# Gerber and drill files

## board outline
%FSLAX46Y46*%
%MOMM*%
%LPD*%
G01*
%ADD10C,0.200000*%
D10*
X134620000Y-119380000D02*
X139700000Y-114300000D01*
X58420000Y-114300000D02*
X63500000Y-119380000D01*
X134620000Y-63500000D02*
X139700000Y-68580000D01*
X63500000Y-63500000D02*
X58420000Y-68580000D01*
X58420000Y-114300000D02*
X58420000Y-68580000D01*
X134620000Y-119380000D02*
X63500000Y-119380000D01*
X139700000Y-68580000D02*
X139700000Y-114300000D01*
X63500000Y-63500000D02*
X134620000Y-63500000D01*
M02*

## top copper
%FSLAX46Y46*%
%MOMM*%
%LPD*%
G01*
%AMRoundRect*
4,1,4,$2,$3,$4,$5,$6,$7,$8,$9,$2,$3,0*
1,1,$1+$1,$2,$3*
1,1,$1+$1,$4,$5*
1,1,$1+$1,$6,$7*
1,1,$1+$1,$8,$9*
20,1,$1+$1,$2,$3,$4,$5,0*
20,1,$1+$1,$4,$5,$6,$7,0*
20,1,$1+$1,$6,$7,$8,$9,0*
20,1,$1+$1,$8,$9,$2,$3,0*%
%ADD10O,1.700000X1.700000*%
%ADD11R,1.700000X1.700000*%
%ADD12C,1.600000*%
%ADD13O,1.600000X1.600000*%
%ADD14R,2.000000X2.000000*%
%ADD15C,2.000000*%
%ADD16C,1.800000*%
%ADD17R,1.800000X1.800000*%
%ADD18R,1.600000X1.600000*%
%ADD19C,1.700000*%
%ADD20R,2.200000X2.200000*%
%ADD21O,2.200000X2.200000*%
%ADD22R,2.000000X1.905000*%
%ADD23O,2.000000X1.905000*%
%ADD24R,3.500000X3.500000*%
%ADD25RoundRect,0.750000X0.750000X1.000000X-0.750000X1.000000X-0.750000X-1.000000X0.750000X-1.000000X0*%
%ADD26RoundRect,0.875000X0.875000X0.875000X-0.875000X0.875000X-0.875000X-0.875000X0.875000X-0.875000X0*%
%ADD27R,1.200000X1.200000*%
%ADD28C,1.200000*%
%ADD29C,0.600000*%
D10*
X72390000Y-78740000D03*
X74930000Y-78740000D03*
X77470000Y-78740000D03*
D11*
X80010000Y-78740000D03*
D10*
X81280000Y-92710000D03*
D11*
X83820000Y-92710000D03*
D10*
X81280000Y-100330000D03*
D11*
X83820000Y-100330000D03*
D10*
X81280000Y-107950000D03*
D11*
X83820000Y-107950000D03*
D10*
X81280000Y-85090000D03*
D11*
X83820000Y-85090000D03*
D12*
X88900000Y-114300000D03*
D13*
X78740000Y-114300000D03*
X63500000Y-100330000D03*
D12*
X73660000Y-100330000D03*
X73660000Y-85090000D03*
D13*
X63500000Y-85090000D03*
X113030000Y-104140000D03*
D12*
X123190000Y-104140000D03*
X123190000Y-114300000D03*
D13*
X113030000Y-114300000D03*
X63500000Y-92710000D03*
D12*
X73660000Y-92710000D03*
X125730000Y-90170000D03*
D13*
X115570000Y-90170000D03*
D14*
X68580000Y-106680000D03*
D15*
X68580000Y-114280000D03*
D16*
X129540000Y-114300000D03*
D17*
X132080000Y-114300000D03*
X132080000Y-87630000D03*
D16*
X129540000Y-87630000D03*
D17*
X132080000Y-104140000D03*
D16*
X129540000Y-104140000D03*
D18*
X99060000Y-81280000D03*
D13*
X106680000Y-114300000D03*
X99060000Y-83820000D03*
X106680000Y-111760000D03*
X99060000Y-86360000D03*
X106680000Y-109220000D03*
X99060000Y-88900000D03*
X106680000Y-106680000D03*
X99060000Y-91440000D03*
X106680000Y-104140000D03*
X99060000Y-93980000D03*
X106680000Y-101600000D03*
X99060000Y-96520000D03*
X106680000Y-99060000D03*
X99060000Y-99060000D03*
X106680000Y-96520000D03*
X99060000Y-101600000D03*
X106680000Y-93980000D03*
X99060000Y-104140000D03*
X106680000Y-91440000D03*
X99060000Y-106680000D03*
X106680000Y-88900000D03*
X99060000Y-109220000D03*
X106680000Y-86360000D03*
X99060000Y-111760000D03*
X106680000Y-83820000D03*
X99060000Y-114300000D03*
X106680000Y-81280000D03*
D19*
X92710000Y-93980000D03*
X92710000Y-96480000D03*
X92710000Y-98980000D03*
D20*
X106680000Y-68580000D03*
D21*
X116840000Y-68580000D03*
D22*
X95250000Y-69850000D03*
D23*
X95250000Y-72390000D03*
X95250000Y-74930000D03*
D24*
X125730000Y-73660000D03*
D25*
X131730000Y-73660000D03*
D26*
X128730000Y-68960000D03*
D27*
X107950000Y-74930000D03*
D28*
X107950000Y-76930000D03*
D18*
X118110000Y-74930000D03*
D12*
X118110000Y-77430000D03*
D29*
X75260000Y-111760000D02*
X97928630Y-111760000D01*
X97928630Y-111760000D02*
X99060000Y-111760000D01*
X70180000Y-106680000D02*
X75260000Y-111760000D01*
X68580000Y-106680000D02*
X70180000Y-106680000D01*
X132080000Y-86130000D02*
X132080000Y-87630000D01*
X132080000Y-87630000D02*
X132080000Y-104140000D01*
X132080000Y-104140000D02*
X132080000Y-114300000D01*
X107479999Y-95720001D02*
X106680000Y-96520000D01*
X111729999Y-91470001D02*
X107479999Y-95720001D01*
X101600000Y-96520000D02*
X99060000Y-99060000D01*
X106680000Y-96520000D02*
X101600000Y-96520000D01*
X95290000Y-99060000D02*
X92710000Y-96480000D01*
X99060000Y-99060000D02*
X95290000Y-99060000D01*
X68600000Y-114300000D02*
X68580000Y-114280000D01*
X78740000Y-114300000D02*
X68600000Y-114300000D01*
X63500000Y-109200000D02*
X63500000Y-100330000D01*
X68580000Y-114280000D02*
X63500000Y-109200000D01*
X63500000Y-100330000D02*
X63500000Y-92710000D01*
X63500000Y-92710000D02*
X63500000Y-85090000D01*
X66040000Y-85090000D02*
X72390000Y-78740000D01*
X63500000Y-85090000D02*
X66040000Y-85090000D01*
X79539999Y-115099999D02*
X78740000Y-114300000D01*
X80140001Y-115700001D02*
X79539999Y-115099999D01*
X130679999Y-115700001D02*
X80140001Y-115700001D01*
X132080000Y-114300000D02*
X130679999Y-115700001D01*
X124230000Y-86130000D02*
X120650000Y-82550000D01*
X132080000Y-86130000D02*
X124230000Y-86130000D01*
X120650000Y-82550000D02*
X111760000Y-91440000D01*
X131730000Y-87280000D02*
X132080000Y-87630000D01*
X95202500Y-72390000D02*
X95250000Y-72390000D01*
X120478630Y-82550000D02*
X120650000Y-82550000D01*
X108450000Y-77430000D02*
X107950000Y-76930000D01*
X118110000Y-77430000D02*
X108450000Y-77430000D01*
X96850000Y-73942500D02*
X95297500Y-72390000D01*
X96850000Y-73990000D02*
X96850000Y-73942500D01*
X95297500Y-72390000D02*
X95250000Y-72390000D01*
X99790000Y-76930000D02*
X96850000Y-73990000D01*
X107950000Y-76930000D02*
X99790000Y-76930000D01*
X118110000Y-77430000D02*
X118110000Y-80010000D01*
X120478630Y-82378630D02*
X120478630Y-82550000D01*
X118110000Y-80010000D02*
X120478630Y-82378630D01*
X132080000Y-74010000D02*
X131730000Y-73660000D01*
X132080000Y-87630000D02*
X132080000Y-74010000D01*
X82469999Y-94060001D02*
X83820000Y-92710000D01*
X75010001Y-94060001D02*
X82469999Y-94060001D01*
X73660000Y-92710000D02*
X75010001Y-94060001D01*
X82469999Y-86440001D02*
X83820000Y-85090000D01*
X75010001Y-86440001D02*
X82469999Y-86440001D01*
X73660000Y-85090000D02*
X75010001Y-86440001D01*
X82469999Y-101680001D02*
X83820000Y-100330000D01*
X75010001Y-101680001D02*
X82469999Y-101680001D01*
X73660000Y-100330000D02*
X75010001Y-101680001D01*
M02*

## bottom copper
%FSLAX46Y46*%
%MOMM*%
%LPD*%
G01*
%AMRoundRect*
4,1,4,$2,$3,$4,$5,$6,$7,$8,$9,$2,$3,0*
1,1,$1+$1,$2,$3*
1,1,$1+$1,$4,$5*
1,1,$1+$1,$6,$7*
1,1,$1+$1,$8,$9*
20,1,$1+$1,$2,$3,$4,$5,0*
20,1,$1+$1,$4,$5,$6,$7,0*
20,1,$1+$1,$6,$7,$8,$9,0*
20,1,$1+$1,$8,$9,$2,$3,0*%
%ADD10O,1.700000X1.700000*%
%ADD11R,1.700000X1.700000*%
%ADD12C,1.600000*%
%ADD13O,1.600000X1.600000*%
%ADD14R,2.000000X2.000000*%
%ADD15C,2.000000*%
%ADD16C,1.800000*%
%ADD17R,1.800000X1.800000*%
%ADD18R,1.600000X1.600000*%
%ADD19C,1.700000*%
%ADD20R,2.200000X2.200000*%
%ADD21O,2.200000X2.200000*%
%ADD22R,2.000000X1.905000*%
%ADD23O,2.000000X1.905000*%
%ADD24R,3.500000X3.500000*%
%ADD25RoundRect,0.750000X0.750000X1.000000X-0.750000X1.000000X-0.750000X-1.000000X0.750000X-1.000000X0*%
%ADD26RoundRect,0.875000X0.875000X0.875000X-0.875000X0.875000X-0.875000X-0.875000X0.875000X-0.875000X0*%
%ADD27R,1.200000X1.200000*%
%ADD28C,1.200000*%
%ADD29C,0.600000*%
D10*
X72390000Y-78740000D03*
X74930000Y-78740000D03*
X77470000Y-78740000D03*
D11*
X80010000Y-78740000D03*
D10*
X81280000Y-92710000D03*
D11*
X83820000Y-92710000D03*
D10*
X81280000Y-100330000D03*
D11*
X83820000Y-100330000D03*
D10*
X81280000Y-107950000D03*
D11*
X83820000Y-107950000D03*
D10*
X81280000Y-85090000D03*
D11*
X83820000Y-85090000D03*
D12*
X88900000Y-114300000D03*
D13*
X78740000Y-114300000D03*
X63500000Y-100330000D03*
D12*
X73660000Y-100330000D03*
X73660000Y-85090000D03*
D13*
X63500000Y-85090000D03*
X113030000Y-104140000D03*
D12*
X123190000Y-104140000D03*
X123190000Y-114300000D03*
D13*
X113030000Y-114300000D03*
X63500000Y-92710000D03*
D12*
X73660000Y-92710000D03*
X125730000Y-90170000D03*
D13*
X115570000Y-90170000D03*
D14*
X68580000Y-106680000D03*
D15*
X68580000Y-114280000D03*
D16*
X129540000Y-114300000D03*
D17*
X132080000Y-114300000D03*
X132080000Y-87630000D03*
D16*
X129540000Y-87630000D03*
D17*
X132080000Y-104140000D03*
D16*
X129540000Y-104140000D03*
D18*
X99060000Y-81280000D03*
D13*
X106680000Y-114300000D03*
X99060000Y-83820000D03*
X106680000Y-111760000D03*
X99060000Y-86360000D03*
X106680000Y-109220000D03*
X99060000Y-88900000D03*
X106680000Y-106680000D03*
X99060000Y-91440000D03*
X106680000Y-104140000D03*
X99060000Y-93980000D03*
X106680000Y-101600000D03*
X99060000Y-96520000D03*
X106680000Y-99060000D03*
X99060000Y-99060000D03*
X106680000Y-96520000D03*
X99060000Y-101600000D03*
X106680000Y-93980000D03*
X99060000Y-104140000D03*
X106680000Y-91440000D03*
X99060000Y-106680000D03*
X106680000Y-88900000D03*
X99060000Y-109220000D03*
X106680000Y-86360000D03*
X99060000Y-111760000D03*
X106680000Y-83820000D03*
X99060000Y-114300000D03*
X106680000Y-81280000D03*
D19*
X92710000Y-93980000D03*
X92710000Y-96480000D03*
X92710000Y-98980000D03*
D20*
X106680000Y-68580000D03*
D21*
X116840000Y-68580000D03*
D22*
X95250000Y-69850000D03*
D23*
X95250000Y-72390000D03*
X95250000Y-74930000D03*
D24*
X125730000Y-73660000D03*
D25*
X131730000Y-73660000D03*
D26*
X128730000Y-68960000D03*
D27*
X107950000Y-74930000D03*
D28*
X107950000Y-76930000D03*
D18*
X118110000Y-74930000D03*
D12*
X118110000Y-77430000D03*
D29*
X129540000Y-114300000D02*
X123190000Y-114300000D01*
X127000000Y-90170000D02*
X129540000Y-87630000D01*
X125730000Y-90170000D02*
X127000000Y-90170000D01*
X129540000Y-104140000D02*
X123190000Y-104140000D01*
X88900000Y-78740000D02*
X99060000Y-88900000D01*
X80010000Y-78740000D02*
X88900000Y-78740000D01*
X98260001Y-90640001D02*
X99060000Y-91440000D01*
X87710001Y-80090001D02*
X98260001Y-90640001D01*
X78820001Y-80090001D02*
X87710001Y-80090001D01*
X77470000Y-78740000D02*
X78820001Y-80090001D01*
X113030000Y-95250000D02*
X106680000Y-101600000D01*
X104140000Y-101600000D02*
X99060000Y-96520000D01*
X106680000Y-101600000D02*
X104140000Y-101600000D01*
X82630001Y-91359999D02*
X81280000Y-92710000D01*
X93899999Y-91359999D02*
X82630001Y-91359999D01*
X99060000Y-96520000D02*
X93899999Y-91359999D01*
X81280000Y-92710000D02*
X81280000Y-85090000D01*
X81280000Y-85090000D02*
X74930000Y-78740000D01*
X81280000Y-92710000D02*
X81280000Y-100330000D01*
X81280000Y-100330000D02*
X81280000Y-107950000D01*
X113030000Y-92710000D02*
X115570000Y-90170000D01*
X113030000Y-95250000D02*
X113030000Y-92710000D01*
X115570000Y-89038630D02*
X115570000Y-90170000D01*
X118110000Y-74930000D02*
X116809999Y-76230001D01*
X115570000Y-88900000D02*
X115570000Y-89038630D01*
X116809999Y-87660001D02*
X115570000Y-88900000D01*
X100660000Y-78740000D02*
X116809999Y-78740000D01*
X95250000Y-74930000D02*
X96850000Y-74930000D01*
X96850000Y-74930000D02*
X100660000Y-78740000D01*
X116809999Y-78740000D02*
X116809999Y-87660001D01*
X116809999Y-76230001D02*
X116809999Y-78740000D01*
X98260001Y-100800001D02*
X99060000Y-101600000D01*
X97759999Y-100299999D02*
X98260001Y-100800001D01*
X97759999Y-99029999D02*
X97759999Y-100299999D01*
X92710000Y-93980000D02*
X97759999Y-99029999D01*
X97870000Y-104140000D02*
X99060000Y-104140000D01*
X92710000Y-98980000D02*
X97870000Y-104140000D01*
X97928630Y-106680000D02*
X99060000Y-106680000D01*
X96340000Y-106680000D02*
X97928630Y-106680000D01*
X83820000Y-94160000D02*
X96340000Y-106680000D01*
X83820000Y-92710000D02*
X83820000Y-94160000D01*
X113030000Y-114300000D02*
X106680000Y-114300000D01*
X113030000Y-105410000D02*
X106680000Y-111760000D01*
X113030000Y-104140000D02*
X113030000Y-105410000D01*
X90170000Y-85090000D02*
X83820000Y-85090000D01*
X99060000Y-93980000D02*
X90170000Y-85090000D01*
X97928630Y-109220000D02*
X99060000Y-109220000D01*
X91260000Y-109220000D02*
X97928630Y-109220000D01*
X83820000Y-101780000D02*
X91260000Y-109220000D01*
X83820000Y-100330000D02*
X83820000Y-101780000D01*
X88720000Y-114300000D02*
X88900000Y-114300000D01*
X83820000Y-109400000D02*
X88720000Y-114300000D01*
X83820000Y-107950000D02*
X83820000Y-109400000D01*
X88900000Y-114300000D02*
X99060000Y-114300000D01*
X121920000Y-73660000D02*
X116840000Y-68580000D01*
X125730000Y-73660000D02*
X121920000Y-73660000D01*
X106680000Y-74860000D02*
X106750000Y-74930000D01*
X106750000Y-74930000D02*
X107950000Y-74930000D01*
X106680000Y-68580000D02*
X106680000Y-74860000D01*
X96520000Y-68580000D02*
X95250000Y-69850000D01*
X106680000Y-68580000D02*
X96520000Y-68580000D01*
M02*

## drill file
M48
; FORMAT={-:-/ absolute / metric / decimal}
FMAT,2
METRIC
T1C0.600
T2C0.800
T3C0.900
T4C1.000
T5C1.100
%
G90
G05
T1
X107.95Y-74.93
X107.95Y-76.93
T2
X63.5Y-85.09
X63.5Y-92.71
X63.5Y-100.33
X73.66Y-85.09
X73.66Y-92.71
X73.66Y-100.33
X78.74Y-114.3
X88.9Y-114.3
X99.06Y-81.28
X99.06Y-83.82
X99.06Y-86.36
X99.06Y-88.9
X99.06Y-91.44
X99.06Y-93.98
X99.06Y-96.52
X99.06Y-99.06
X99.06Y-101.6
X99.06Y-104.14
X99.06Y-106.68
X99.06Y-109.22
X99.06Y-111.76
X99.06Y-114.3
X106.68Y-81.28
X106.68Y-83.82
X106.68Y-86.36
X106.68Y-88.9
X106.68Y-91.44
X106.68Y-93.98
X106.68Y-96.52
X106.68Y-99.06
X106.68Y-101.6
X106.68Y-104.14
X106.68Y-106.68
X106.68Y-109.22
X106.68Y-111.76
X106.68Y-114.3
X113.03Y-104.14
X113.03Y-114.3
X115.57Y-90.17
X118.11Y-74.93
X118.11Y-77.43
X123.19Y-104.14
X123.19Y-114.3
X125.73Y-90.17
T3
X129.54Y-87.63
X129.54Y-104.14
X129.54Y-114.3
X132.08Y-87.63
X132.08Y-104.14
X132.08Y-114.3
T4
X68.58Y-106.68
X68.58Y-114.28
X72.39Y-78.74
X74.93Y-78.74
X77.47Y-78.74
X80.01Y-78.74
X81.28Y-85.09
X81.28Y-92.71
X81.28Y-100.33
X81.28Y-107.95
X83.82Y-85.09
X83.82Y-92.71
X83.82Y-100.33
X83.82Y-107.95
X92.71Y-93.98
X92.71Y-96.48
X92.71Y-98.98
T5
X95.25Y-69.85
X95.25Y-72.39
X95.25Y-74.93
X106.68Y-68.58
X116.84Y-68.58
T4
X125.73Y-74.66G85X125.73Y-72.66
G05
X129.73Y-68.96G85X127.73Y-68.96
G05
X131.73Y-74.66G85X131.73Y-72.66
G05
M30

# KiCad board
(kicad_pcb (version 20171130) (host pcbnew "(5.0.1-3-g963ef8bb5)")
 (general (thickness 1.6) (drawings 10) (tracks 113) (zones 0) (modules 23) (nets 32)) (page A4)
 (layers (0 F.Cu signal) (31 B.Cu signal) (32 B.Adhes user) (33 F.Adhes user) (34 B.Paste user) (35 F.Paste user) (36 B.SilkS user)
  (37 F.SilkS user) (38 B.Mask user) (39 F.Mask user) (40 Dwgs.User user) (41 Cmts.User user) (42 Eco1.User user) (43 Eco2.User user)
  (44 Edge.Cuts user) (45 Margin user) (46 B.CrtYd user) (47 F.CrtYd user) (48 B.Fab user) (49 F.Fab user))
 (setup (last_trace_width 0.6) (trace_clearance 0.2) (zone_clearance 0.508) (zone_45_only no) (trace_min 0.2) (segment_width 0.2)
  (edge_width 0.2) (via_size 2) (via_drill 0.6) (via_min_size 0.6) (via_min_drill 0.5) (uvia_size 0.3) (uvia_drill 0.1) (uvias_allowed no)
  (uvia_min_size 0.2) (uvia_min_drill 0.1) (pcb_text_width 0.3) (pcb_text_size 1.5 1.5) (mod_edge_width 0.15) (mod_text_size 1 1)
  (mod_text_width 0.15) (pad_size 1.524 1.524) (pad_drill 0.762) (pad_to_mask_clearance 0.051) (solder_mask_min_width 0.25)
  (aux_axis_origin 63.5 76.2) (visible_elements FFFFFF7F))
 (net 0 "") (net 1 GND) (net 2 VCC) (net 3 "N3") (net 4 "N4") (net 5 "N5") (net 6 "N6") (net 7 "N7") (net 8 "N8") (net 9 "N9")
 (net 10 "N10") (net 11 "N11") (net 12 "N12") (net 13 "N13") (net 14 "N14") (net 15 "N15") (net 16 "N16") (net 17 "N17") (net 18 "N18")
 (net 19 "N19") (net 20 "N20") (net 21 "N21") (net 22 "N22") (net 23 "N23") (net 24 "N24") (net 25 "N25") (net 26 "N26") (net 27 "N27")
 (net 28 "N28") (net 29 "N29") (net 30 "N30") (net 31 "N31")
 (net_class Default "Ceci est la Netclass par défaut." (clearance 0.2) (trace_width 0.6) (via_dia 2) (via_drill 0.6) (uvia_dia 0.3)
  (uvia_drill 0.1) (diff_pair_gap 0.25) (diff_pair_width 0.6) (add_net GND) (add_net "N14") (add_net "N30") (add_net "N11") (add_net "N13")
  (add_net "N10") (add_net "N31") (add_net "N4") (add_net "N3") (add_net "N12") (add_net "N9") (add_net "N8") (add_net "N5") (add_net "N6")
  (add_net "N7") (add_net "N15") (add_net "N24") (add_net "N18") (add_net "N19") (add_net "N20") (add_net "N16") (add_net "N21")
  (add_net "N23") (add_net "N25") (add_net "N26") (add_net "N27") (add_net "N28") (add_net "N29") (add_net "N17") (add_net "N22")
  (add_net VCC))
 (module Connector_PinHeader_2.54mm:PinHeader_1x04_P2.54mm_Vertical (layer F.Cu) (at 80.01 78.74 270)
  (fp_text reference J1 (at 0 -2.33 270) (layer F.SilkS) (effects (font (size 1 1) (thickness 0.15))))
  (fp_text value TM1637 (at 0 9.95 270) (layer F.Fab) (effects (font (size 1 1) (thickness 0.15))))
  (pad 4 thru_hole oval (at 0 7.62 270) (size 1.7 1.7) (drill 1) (layers *.Cu *.Mask) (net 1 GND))
  (pad 3 thru_hole oval (at 0 5.08 270) (size 1.7 1.7) (drill 1) (layers *.Cu *.Mask) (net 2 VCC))
  (pad 2 thru_hole oval (at 0 2.54 270) (size 1.7 1.7) (drill 1) (layers *.Cu *.Mask) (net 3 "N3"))
  (pad 1 thru_hole rect (at 0 0 270) (size 1.7 1.7) (drill 1) (layers *.Cu *.Mask) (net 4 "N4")))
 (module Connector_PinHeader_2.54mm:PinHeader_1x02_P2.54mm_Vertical (layer F.Cu) (at 83.82 92.71 270)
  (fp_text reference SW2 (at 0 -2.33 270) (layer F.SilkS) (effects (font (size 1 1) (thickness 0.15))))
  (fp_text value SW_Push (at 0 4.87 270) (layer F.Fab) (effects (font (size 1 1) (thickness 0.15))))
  (pad 2 thru_hole oval (at 0 2.54 270) (size 1.7 1.7) (drill 1) (layers *.Cu *.Mask) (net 2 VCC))
  (pad 1 thru_hole rect (at 0 0 270) (size 1.7 1.7) (drill 1) (layers *.Cu *.Mask) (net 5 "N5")))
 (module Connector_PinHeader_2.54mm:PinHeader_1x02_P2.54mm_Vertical (layer F.Cu) (at 83.82 100.33 270)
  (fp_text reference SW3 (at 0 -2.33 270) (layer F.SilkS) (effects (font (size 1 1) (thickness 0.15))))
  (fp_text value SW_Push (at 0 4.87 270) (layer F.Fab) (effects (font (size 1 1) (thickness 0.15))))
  (pad 2 thru_hole oval (at 0 2.54 270) (size 1.7 1.7) (drill 1) (layers *.Cu *.Mask) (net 2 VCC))
  (pad 1 thru_hole rect (at 0 0 270) (size 1.7 1.7) (drill 1) (layers *.Cu *.Mask) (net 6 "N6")))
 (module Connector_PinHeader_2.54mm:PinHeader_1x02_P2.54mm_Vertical (layer F.Cu) (at 83.82 107.95 270)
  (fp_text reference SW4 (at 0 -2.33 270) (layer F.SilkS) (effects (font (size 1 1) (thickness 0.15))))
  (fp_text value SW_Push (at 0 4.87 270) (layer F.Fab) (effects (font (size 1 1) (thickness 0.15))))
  (pad 2 thru_hole oval (at 0 2.54 270) (size 1.7 1.7) (drill 1) (layers *.Cu *.Mask) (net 2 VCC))
  (pad 1 thru_hole rect (at 0 0 270) (size 1.7 1.7) (drill 1) (layers *.Cu *.Mask) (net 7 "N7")))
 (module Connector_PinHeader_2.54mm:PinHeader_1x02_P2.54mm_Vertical (layer F.Cu) (at 83.82 85.09 270)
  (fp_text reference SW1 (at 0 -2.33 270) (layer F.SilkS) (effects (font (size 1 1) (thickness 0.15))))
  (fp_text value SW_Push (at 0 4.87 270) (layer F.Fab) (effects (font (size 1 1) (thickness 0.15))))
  (pad 2 thru_hole oval (at 0 2.54 270) (size 1.7 1.7) (drill 1) (layers *.Cu *.Mask) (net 2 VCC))
  (pad 1 thru_hole rect (at 0 0 270) (size 1.7 1.7) (drill 1) (layers *.Cu *.Mask) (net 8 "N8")))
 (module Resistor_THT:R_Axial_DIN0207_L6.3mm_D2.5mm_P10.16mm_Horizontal (layer F.Cu) (at 88.9 114.3 180)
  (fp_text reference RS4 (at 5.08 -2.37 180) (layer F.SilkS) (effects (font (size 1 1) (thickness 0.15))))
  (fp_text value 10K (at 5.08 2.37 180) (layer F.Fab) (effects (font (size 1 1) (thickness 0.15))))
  (pad 1 thru_hole circle (at 0 0 180) (size 1.6 1.6) (drill 0.8) (layers *.Cu *.Mask) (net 7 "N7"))
  (pad 2 thru_hole oval (at 10.16 0 180) (size 1.6 1.6) (drill 0.8) (layers *.Cu *.Mask) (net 1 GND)))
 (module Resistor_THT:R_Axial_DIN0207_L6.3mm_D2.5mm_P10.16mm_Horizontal (layer F.Cu) (at 73.66 100.33 180)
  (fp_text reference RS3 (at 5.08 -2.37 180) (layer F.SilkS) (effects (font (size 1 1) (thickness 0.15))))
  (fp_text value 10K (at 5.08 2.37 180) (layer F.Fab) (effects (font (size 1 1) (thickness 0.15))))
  (pad 2 thru_hole oval (at 10.16 0 180) (size 1.6 1.6) (drill 0.8) (layers *.Cu *.Mask) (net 1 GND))
  (pad 1 thru_hole circle (at 0 0 180) (size 1.6 1.6) (drill 0.8) (layers *.Cu *.Mask) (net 6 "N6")))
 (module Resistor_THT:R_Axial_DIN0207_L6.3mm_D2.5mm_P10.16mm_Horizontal (layer F.Cu) (at 73.66 85.09 180)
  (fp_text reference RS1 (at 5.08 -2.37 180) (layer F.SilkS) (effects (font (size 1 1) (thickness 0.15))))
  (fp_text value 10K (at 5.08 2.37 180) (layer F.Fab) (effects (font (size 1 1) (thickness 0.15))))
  (pad 1 thru_hole circle (at 0 0 180) (size 1.6 1.6) (drill 0.8) (layers *.Cu *.Mask) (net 8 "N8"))
  (pad 2 thru_hole oval (at 10.16 0 180) (size 1.6 1.6) (drill 0.8) (layers *.Cu *.Mask) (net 1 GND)))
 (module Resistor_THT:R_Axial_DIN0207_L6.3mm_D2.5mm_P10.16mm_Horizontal (layer F.Cu) (at 123.19 104.14 180)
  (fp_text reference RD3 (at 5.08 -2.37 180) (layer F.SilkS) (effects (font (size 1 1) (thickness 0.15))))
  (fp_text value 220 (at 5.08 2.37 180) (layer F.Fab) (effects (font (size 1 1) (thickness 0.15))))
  (pad 2 thru_hole oval (at 10.16 0 180) (size 1.6 1.6) (drill 0.8) (layers *.Cu *.Mask) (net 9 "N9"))
  (pad 1 thru_hole circle (at 0 0 180) (size 1.6 1.6) (drill 0.8) (layers *.Cu *.Mask) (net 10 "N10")))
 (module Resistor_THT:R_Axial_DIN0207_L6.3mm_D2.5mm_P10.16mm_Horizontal (layer F.Cu) (at 123.19 114.3 180)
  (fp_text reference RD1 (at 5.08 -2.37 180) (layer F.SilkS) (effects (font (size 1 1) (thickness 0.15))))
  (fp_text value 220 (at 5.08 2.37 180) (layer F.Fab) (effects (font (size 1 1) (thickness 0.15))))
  (pad 1 thru_hole circle (at 0 0 180) (size 1.6 1.6) (drill 0.8) (layers *.Cu *.Mask) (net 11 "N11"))
  (pad 2 thru_hole oval (at 10.16 0 180) (size 1.6 1.6) (drill 0.8) (layers *.Cu *.Mask) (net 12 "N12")))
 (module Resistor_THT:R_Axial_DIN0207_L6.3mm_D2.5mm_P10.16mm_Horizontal (layer F.Cu) (at 73.66 92.71 180)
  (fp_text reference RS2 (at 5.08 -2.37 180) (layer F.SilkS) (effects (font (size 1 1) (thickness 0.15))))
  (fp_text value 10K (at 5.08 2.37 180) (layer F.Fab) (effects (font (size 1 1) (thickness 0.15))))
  (pad 2 thru_hole oval (at 10.16 0 180) (size 1.6 1.6) (drill 0.8) (layers *.Cu *.Mask) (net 1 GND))
  (pad 1 thru_hole circle (at 0 0 180) (size 1.6 1.6) (drill 0.8) (layers *.Cu *.Mask) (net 5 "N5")))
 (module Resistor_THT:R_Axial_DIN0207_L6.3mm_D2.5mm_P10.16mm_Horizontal (layer F.Cu) (at 125.73 90.17 180)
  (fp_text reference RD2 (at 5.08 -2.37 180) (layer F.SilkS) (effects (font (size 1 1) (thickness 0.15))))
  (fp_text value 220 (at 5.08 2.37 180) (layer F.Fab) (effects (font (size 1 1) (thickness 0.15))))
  (pad 1 thru_hole circle (at 0 0 180) (size 1.6 1.6) (drill 0.8) (layers *.Cu *.Mask) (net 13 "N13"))
  (pad 2 thru_hole oval (at 10.16 0 180) (size 1.6 1.6) (drill 0.8) (layers *.Cu *.Mask) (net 2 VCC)))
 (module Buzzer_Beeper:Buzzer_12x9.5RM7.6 (layer F.Cu) (at 68.58 106.68 270)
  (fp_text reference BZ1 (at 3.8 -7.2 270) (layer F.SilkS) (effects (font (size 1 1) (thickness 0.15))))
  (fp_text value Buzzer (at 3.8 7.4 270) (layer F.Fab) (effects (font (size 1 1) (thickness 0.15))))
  (pad 1 thru_hole rect (at 0 0 270) (size 2 2) (drill 1) (layers *.Cu *.Mask) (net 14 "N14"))
  (pad 2 thru_hole circle (at 7.6 0 270) (size 2 2) (drill 1) (layers *.Cu *.Mask) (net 1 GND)))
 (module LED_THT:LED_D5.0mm (layer F.Cu) (at 132.08 114.3 180)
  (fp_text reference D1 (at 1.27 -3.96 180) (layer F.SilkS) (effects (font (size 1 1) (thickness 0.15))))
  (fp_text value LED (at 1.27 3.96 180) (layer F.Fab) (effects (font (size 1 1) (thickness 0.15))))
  (pad 2 thru_hole circle (at 2.54 0 180) (size 1.8 1.8) (drill 0.9) (layers *.Cu *.Mask) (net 11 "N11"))
  (pad 1 thru_hole rect (at 0 0 180) (size 1.8 1.8) (drill 0.9) (layers *.Cu *.Mask) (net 1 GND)))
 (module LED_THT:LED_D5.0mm (layer F.Cu) (at 132.08 87.63 180)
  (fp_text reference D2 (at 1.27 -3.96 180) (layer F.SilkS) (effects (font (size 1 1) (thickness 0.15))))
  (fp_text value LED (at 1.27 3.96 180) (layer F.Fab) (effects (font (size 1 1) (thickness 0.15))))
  (pad 1 thru_hole rect (at 0 0 180) (size 1.8 1.8) (drill 0.9) (layers *.Cu *.Mask) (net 1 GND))
  (pad 2 thru_hole circle (at 2.54 0 180) (size 1.8 1.8) (drill 0.9) (layers *.Cu *.Mask) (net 13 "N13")))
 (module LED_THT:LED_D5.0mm (layer F.Cu) (at 132.08 104.14 180)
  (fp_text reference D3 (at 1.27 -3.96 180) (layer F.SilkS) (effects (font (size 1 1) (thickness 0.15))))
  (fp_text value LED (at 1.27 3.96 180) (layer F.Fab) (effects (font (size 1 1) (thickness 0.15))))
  (pad 1 thru_hole rect (at 0 0 180) (size 1.8 1.8) (drill 0.9) (layers *.Cu *.Mask) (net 1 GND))
  (pad 2 thru_hole circle (at 2.54 0 180) (size 1.8 1.8) (drill 0.9) (layers *.Cu *.Mask) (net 10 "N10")))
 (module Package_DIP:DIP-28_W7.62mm (layer F.Cu) (at 99.06 81.28)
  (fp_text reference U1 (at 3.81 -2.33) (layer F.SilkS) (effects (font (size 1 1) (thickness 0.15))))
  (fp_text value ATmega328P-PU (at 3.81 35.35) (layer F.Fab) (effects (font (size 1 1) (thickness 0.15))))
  (pad 1 thru_hole rect (at 0 0) (size 1.6 1.6) (drill 0.8) (layers *.Cu *.Mask) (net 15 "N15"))
  (pad 15 thru_hole oval (at 7.62 33.02) (size 1.6 1.6) (drill 0.8) (layers *.Cu *.Mask) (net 12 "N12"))
  (pad 2 thru_hole oval (at 0 2.54) (size 1.6 1.6) (drill 0.8) (layers *.Cu *.Mask) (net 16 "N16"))
  (pad 16 thru_hole oval (at 7.62 30.48) (size 1.6 1.6) (drill 0.8) (layers *.Cu *.Mask) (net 9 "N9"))
  (pad 3 thru_hole oval (at 0 5.08) (size 1.6 1.6) (drill 0.8) (layers *.Cu *.Mask) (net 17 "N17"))
  (pad 17 thru_hole oval (at 7.62 27.94) (size 1.6 1.6) (drill 0.8) (layers *.Cu *.Mask) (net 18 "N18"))
  (pad 4 thru_hole oval (at 0 7.62) (size 1.6 1.6) (drill 0.8) (layers *.Cu *.Mask) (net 4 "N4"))
  (pad 18 thru_hole oval (at 7.62 25.4) (size 1.6 1.6) (drill 0.8) (layers *.Cu *.Mask) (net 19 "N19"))
  (pad 5 thru_hole oval (at 0 10.16) (size 1.6 1.6) (drill 0.8) (layers *.Cu *.Mask) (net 3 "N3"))
  (pad 19 thru_hole oval (at 7.62 22.86) (size 1.6 1.6) (drill 0.8) (layers *.Cu *.Mask) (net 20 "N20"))
  (pad 6 thru_hole oval (at 0 12.7) (size 1.6 1.6) (drill 0.8) (layers *.Cu *.Mask) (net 8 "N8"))
  (pad 20 thru_hole oval (at 7.62 20.32) (size 1.6 1.6) (drill 0.8) (layers *.Cu *.Mask) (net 2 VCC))
  (pad 7 thru_hole oval (at 0 15.24) (size 1.6 1.6) (drill 0.8) (layers *.Cu *.Mask) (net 2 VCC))
  (pad 21 thru_hole oval (at 7.62 17.78) (size 1.6 1.6) (drill 0.8) (layers *.Cu *.Mask) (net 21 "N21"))
  (pad 8 thru_hole oval (at 0 17.78) (size 1.6 1.6) (drill 0.8) (layers *.Cu *.Mask) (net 1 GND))
  (pad 22 thru_hole oval (at 7.62 15.24) (size 1.6 1.6) (drill 0.8) (layers *.Cu *.Mask) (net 1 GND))
  (pad 9 thru_hole oval (at 0 20.32) (size 1.6 1.6) (drill 0.8) (layers *.Cu *.Mask) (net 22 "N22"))
  (pad 23 thru_hole oval (at 7.62 12.7) (size 1.6 1.6) (drill 0.8) (layers *.Cu *.Mask) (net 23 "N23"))
  (pad 10 thru_hole oval (at 0 22.86) (size 1.6 1.6) (drill 0.8) (layers *.Cu *.Mask) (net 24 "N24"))
  (pad 24 thru_hole oval (at 7.62 10.16) (size 1.6 1.6) (drill 0.8) (layers *.Cu *.Mask) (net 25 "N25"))
  (pad 11 thru_hole oval (at 0 25.4) (size 1.6 1.6) (drill 0.8) (layers *.Cu *.Mask) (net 5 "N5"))
  (pad 25 thru_hole oval (at 7.62 7.62) (size 1.6 1.6) (drill 0.8) (layers *.Cu *.Mask) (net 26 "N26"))
  (pad 12 thru_hole oval (at 0 27.94) (size 1.6 1.6) (drill 0.8) (layers *.Cu *.Mask) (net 6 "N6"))
  (pad 26 thru_hole oval (at 7.62 5.08) (size 1.6 1.6) (drill 0.8) (layers *.Cu *.Mask) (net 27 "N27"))
  (pad 13 thru_hole oval (at 0 30.48) (size 1.6 1.6) (drill 0.8) (layers *.Cu *.Mask) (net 14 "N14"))
  (pad 27 thru_hole oval (at 7.62 2.54) (size 1.6 1.6) (drill 0.8) (layers *.Cu *.Mask) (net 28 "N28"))
  (pad 14 thru_hole oval (at 0 33.02) (size 1.6 1.6) (drill 0.8) (layers *.Cu *.Mask) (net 7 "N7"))
  (pad 28 thru_hole oval (at 7.62 0) (size 1.6 1.6) (drill 0.8) (layers *.Cu *.Mask) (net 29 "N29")))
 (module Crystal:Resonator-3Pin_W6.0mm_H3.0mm (layer F.Cu) (at 92.71 93.98 270)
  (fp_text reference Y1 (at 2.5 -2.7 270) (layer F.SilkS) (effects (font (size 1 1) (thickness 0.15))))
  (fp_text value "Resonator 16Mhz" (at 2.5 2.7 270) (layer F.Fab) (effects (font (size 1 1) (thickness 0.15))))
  (pad 1 thru_hole circle (at 0 0 270) (size 1.7 1.7) (drill 1) (layers *.Cu *.Mask) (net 22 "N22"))
  (pad 2 thru_hole circle (at 2.5 0 270) (size 1.7 1.7) (drill 1) (layers *.Cu *.Mask) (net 1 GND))
  (pad 3 thru_hole circle (at 5 0 270) (size 1.7 1.7) (drill 1) (layers *.Cu *.Mask) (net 24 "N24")))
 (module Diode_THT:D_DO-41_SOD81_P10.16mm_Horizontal (layer F.Cu) (at 106.68 68.58)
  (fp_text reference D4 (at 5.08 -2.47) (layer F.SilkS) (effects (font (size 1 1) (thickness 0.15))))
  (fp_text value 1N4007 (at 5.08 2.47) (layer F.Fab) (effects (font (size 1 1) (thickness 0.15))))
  (pad 1 thru_hole rect (at 0 0) (size 2.2 2.2) (drill 1.1) (layers *.Cu *.Mask) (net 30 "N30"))
  (pad 2 thru_hole oval (at 10.16 0) (size 2.2 2.2) (drill 1.1) (layers *.Cu *.Mask) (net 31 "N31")))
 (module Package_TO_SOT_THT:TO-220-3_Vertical (layer F.Cu) (at 95.25 69.85 270)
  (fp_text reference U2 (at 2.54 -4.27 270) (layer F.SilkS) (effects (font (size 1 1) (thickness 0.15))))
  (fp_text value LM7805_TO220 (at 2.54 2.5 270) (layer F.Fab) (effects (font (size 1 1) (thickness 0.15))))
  (pad 1 thru_hole rect (at 0 0 270) (size 1.905 2) (drill 1.1) (layers *.Cu *.Mask) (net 30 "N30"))
  (pad 2 thru_hole oval (at 2.54 0 270) (size 1.905 2) (drill 1.1) (layers *.Cu *.Mask) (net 1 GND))
  (pad 3 thru_hole oval (at 5.08 0 270) (size 1.905 2) (drill 1.1) (layers *.Cu *.Mask) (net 2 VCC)))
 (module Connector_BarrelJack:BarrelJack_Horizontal (layer F.Cu) (at 125.73 73.66 180)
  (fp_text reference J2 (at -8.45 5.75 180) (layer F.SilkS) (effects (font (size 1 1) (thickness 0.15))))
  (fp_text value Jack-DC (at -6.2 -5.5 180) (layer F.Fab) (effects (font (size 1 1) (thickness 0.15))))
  (pad 1 thru_hole rect (at 0 0 180) (size 3.5 3.5) (drill oval 1 3) (layers *.Cu *.Mask) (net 31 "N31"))
  (pad 2 thru_hole roundrect (at -6 0 180) (size 3 3.5) (drill oval 1 3) (layers *.Cu *.Mask) (roundrect_rratio 0.25) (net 1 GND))
  (pad 3 thru_hole roundrect (at -3 4.7 180) (size 3.5 3.5) (drill oval 3 1) (layers *.Cu *.Mask) (roundrect_rratio 0.25)))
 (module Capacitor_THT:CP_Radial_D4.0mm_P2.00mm (layer F.Cu) (at 107.95 74.93 270)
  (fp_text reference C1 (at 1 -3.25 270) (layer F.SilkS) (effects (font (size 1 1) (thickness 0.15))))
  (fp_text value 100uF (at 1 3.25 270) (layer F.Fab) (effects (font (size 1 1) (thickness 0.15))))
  (pad 1 thru_hole rect (at 0 0 270) (size 1.2 1.2) (drill 0.6) (layers *.Cu *.Mask) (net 30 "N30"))
  (pad 2 thru_hole circle (at 2 0 270) (size 1.2 1.2) (drill 0.6) (layers *.Cu *.Mask) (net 1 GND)))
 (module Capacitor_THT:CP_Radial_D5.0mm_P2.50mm (layer F.Cu) (at 118.11 74.93 270)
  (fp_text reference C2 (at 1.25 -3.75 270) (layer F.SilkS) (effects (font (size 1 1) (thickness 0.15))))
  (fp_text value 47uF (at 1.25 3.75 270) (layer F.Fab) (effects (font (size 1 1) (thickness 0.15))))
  (pad 1 thru_hole rect (at 0 0 270) (size 1.6 1.6) (drill 0.8) (layers *.Cu *.Mask) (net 2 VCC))
  (pad 2 thru_hole circle (at 2.5 0 270) (size 1.6 1.6) (drill 0.8) (layers *.Cu *.Mask) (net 1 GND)))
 (gr_line (start 134.62 119.38) (end 139.7 114.3) (layer Edge.Cuts) (width 0.2))
 (gr_line (start 58.42 114.3) (end 63.5 119.38) (layer Edge.Cuts) (width 0.2))
 (gr_line (start 134.62 63.5) (end 139.7 68.58) (layer Edge.Cuts) (width 0.2))
 (gr_line (start 63.5 63.5) (end 58.42 68.58) (layer Edge.Cuts) (width 0.2))
 (gr_line (start 58.42 114.3) (end 58.42 68.58) (layer Edge.Cuts) (width 0.2))
 (gr_line (start 134.62 119.38) (end 63.5 119.38) (layer Edge.Cuts) (width 0.2))
 (gr_line (start 139.7 68.58) (end 139.7 114.3) (layer Edge.Cuts) (width 0.2))
 (gr_line (start 63.5 63.5) (end 134.62 63.5) (layer Edge.Cuts) (width 0.2))
 (segment (start 75.26 111.76) (end 97.92863 111.76) (width 0.6) (layer F.Cu) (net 14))
 (segment (start 97.92863 111.76) (end 99.06 111.76) (width 0.6) (layer F.Cu) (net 14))
 (segment (start 70.18 106.68) (end 75.26 111.76) (width 0.6) (layer F.Cu) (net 14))
 (segment (start 68.58 106.68) (end 70.18 106.68) (width 0.6) (layer F.Cu) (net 14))
 (segment (start 132.08 86.13) (end 132.08 87.63) (width 0.6) (layer F.Cu) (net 1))
 (segment (start 132.08 87.63) (end 132.08 104.14) (width 0.6) (layer F.Cu) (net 1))
 (segment (start 132.08 104.14) (end 132.08 114.3) (width 0.6) (layer F.Cu) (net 1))
 (segment (start 107.479999 95.720001) (end 106.68 96.52) (width 0.6) (layer F.Cu) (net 1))
 (segment (start 111.729999 91.470001) (end 107.479999 95.720001) (width 0.6) (layer F.Cu) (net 1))
 (segment (start 101.6 96.52) (end 99.06 99.06) (width 0.6) (layer F.Cu) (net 1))
 (segment (start 106.68 96.52) (end 101.6 96.52) (width 0.6) (layer F.Cu) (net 1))
 (segment (start 95.29 99.06) (end 92.71 96.48) (width 0.6) (layer F.Cu) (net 1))
 (segment (start 99.06 99.06) (end 95.29 99.06) (width 0.6) (layer F.Cu) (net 1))
 (segment (start 68.6 114.3) (end 68.58 114.28) (width 0.6) (layer F.Cu) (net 1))
 (segment (start 78.74 114.3) (end 68.6 114.3) (width 0.6) (layer F.Cu) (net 1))
 (segment (start 63.5 109.2) (end 63.5 100.33) (width 0.6) (layer F.Cu) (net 1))
 (segment (start 68.58 114.28) (end 63.5 109.2) (width 0.6) (layer F.Cu) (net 1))
 (segment (start 63.5 100.33) (end 63.5 92.71) (width 0.6) (layer F.Cu) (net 1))
 (segment (start 63.5 92.71) (end 63.5 85.09) (width 0.6) (layer F.Cu) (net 1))
 (segment (start 66.04 85.09) (end 72.39 78.74) (width 0.6) (layer F.Cu) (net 1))
 (segment (start 63.5 85.09) (end 66.04 85.09) (width 0.6) (layer F.Cu) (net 1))
 (segment (start 79.539999 115.099999) (end 78.74 114.3) (width 0.6) (layer F.Cu) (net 1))
 (segment (start 80.140001 115.700001) (end 79.539999 115.099999) (width 0.6) (layer F.Cu) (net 1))
 (segment (start 130.679999 115.700001) (end 80.140001 115.700001) (width 0.6) (layer F.Cu) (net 1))
 (segment (start 132.08 114.3) (end 130.679999 115.700001) (width 0.6) (layer F.Cu) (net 1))
 (segment (start 124.23 86.13) (end 120.65 82.55) (width 0.6) (layer F.Cu) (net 1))
 (segment (start 132.08 86.13) (end 124.23 86.13) (width 0.6) (layer F.Cu) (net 1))
 (segment (start 120.65 82.55) (end 111.76 91.44) (width 0.6) (layer F.Cu) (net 1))
 (segment (start 131.73 87.28) (end 132.08 87.63) (width 0.6) (layer F.Cu) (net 1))
 (segment (start 95.2025 72.39) (end 95.25 72.39) (width 0.6) (layer F.Cu) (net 1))
 (segment (start 120.47863 82.55) (end 120.65 82.55) (width 0.6) (layer F.Cu) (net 1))
 (segment (start 108.45 77.43) (end 107.95 76.93) (width 0.6) (layer F.Cu) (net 1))
 (segment (start 118.11 77.43) (end 108.45 77.43) (width 0.6) (layer F.Cu) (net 1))
 (segment (start 96.85 73.9425) (end 95.2975 72.39) (width 0.6) (layer F.Cu) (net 1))
 (segment (start 96.85 73.99) (end 96.85 73.9425) (width 0.6) (layer F.Cu) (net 1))
 (segment (start 95.2975 72.39) (end 95.25 72.39) (width 0.6) (layer F.Cu) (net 1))
 (segment (start 99.79 76.93) (end 96.85 73.99) (width 0.6) (layer F.Cu) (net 1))
 (segment (start 107.95 76.93) (end 99.79 76.93) (width 0.6) (layer F.Cu) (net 1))
 (segment (start 118.11 77.43) (end 118.11 80.01) (width 0.6) (layer F.Cu) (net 1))
 (segment (start 120.47863 82.37863) (end 120.47863 82.55) (width 0.6) (layer F.Cu) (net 1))
 (segment (start 118.11 80.01) (end 120.47863 82.37863) (width 0.6) (layer F.Cu) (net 1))
 (segment (start 132.08 74.01) (end 131.73 73.66) (width 0.6) (layer F.Cu) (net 1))
 (segment (start 132.08 87.63) (end 132.08 74.01) (width 0.6) (layer F.Cu) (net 1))
 (segment (start 129.54 114.3) (end 123.19 114.3) (width 0.6) (layer B.Cu) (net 11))
 (segment (start 127 90.17) (end 129.54 87.63) (width 0.6) (layer B.Cu) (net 13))
 (segment (start 125.73 90.17) (end 127 90.17) (width 0.6) (layer B.Cu) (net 13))
 (segment (start 129.54 104.14) (end 123.19 104.14) (width 0.6) (layer B.Cu) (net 10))
 (segment (start 88.9 78.74) (end 99.06 88.9) (width 0.6) (layer B.Cu) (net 4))
 (segment (start 80.01 78.74) (end 88.9 78.74) (width 0.6) (layer B.Cu) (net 4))
 (segment (start 98.260001 90.640001) (end 99.06 91.44) (width 0.6) (layer B.Cu) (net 3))
 (segment (start 87.710001 80.090001) (end 98.260001 90.640001) (width 0.6) (layer B.Cu) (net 3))
 (segment (start 78.820001 80.090001) (end 87.710001 80.090001) (width 0.6) (layer B.Cu) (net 3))
 (segment (start 77.47 78.74) (end 78.820001 80.090001) (width 0.6) (layer B.Cu) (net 3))
 (segment (start 113.03 95.25) (end 106.68 101.6) (width 0.6) (layer B.Cu) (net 2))
 (segment (start 104.14 101.6) (end 99.06 96.52) (width 0.6) (layer B.Cu) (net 2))
 (segment (start 106.68 101.6) (end 104.14 101.6) (width 0.6) (layer B.Cu) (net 2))
 (segment (start 82.630001 91.359999) (end 81.28 92.71) (width 0.6) (layer B.Cu) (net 2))
 (segment (start 93.899999 91.359999) (end 82.630001 91.359999) (width 0.6) (layer B.Cu) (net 2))
 (segment (start 99.06 96.52) (end 93.899999 91.359999) (width 0.6) (layer B.Cu) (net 2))
 (segment (start 81.28 92.71) (end 81.28 85.09) (width 0.6) (layer B.Cu) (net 2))
 (segment (start 81.28 85.09) (end 74.93 78.74) (width 0.6) (layer B.Cu) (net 2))
 (segment (start 81.28 92.71) (end 81.28 100.33) (width 0.6) (layer B.Cu) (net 2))
 (segment (start 81.28 100.33) (end 81.28 107.95) (width 0.6) (layer B.Cu) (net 2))
 (segment (start 113.03 92.71) (end 115.57 90.17) (width 0.6) (layer B.Cu) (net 2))
 (segment (start 113.03 95.25) (end 113.03 92.71) (width 0.6) (layer B.Cu) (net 2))
 (segment (start 115.57 89.03863) (end 115.57 90.17) (width 0.6) (layer B.Cu) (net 2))
 (segment (start 118.11 74.93) (end 116.809999 76.230001) (width 0.6) (layer B.Cu) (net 2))
 (segment (start 115.57 88.9) (end 115.57 89.03863) (width 0.6) (layer B.Cu) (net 2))
 (segment (start 116.809999 87.660001) (end 115.57 88.9) (width 0.6) (layer B.Cu) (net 2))
 (segment (start 100.66 78.74) (end 116.809999 78.74) (width 0.6) (layer B.Cu) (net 2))
 (segment (start 95.25 74.93) (end 96.85 74.93) (width 0.6) (layer B.Cu) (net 2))
 (segment (start 96.85 74.93) (end 100.66 78.74) (width 0.6) (layer B.Cu) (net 2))
 (segment (start 116.809999 78.74) (end 116.809999 87.660001) (width 0.6) (layer B.Cu) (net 2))
 (segment (start 116.809999 76.230001) (end 116.809999 78.74) (width 0.6) (layer B.Cu) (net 2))
 (segment (start 98.260001 100.800001) (end 99.06 101.6) (width 0.6) (layer B.Cu) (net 22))
 (segment (start 97.759999 100.299999) (end 98.260001 100.800001) (width 0.6) (layer B.Cu) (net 22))
 (segment (start 97.759999 99.029999) (end 97.759999 100.299999) (width 0.6) (layer B.Cu) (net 22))
 (segment (start 92.71 93.98) (end 97.759999 99.029999) (width 0.6) (layer B.Cu) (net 22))
 (segment (start 97.87 104.14) (end 99.06 104.14) (width 0.6) (layer B.Cu) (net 24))
 (segment (start 92.71 98.98) (end 97.87 104.14) (width 0.6) (layer B.Cu) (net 24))
 (segment (start 82.469999 94.060001) (end 83.82 92.71) (width 0.6) (layer F.Cu) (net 5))
 (segment (start 75.010001 94.060001) (end 82.469999 94.060001) (width 0.6) (layer F.Cu) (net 5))
 (segment (start 73.66 92.71) (end 75.010001 94.060001) (width 0.6) (layer F.Cu) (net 5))
 (segment (start 97.92863 106.68) (end 99.06 106.68) (width 0.6) (layer B.Cu) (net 5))
 (segment (start 96.34 106.68) (end 97.92863 106.68) (width 0.6) (layer B.Cu) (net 5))
 (segment (start 83.82 94.16) (end 96.34 106.68) (width 0.6) (layer B.Cu) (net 5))
 (segment (start 83.82 92.71) (end 83.82 94.16) (width 0.6) (layer B.Cu) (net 5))
 (segment (start 113.03 114.3) (end 106.68 114.3) (width 0.6) (layer B.Cu) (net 12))
 (segment (start 113.03 105.41) (end 106.68 111.76) (width 0.6) (layer B.Cu) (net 9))
 (segment (start 113.03 104.14) (end 113.03 105.41) (width 0.6) (layer B.Cu) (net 9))
 (segment (start 90.17 85.09) (end 83.82 85.09) (width 0.6) (layer B.Cu) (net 8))
 (segment (start 99.06 93.98) (end 90.17 85.09) (width 0.6) (layer B.Cu) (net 8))
 (segment (start 82.469999 86.440001) (end 83.82 85.09) (width 0.6) (layer F.Cu) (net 8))
 (segment (start 75.010001 86.440001) (end 82.469999 86.440001) (width 0.6) (layer F.Cu) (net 8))
 (segment (start 73.66 85.09) (end 75.010001 86.440001) (width 0.6) (layer F.Cu) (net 8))
 (segment (start 82.469999 101.680001) (end 83.82 100.33) (width 0.6) (layer F.Cu) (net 6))
 (segment (start 75.010001 101.680001) (end 82.469999 101.680001) (width 0.6) (layer F.Cu) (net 6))
 (segment (start 73.66 100.33) (end 75.010001 101.680001) (width 0.6) (layer F.Cu) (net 6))
 (segment (start 97.92863 109.22) (end 99.06 109.22) (width 0.6) (layer B.Cu) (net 6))
 (segment (start 91.26 109.22) (end 97.92863 109.22) (width 0.6) (layer B.Cu) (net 6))
 (segment (start 83.82 101.78) (end 91.26 109.22) (width 0.6) (layer B.Cu) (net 6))
 (segment (start 83.82 100.33) (end 83.82 101.78) (width 0.6) (layer B.Cu) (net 6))
 (segment (start 88.72 114.3) (end 88.9 114.3) (width 0.6) (layer B.Cu) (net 7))
 (segment (start 83.82 109.4) (end 88.72 114.3) (width 0.6) (layer B.Cu) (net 7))
 (segment (start 83.82 107.95) (end 83.82 109.4) (width 0.6) (layer B.Cu) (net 7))
 (segment (start 88.9 114.3) (end 99.06 114.3) (width 0.6) (layer B.Cu) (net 7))
 (segment (start 121.92 73.66) (end 116.84 68.58) (width 0.6) (layer B.Cu) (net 31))
 (segment (start 125.73 73.66) (end 121.92 73.66) (width 0.6) (layer B.Cu) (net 31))
 (segment (start 106.68 74.86) (end 106.75 74.93) (width 0.6) (layer B.Cu) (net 30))
 (segment (start 106.75 74.93) (end 107.95 74.93) (width 0.6) (layer B.Cu) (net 30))
 (segment (start 106.68 68.58) (end 106.68 74.86) (width 0.6) (layer B.Cu) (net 30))
 (segment (start 96.52 68.58) (end 95.25 69.85) (width 0.6) (layer B.Cu) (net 30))
 (segment (start 106.68 68.58) (end 96.52 68.58) (width 0.6) (layer B.Cu) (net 30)))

